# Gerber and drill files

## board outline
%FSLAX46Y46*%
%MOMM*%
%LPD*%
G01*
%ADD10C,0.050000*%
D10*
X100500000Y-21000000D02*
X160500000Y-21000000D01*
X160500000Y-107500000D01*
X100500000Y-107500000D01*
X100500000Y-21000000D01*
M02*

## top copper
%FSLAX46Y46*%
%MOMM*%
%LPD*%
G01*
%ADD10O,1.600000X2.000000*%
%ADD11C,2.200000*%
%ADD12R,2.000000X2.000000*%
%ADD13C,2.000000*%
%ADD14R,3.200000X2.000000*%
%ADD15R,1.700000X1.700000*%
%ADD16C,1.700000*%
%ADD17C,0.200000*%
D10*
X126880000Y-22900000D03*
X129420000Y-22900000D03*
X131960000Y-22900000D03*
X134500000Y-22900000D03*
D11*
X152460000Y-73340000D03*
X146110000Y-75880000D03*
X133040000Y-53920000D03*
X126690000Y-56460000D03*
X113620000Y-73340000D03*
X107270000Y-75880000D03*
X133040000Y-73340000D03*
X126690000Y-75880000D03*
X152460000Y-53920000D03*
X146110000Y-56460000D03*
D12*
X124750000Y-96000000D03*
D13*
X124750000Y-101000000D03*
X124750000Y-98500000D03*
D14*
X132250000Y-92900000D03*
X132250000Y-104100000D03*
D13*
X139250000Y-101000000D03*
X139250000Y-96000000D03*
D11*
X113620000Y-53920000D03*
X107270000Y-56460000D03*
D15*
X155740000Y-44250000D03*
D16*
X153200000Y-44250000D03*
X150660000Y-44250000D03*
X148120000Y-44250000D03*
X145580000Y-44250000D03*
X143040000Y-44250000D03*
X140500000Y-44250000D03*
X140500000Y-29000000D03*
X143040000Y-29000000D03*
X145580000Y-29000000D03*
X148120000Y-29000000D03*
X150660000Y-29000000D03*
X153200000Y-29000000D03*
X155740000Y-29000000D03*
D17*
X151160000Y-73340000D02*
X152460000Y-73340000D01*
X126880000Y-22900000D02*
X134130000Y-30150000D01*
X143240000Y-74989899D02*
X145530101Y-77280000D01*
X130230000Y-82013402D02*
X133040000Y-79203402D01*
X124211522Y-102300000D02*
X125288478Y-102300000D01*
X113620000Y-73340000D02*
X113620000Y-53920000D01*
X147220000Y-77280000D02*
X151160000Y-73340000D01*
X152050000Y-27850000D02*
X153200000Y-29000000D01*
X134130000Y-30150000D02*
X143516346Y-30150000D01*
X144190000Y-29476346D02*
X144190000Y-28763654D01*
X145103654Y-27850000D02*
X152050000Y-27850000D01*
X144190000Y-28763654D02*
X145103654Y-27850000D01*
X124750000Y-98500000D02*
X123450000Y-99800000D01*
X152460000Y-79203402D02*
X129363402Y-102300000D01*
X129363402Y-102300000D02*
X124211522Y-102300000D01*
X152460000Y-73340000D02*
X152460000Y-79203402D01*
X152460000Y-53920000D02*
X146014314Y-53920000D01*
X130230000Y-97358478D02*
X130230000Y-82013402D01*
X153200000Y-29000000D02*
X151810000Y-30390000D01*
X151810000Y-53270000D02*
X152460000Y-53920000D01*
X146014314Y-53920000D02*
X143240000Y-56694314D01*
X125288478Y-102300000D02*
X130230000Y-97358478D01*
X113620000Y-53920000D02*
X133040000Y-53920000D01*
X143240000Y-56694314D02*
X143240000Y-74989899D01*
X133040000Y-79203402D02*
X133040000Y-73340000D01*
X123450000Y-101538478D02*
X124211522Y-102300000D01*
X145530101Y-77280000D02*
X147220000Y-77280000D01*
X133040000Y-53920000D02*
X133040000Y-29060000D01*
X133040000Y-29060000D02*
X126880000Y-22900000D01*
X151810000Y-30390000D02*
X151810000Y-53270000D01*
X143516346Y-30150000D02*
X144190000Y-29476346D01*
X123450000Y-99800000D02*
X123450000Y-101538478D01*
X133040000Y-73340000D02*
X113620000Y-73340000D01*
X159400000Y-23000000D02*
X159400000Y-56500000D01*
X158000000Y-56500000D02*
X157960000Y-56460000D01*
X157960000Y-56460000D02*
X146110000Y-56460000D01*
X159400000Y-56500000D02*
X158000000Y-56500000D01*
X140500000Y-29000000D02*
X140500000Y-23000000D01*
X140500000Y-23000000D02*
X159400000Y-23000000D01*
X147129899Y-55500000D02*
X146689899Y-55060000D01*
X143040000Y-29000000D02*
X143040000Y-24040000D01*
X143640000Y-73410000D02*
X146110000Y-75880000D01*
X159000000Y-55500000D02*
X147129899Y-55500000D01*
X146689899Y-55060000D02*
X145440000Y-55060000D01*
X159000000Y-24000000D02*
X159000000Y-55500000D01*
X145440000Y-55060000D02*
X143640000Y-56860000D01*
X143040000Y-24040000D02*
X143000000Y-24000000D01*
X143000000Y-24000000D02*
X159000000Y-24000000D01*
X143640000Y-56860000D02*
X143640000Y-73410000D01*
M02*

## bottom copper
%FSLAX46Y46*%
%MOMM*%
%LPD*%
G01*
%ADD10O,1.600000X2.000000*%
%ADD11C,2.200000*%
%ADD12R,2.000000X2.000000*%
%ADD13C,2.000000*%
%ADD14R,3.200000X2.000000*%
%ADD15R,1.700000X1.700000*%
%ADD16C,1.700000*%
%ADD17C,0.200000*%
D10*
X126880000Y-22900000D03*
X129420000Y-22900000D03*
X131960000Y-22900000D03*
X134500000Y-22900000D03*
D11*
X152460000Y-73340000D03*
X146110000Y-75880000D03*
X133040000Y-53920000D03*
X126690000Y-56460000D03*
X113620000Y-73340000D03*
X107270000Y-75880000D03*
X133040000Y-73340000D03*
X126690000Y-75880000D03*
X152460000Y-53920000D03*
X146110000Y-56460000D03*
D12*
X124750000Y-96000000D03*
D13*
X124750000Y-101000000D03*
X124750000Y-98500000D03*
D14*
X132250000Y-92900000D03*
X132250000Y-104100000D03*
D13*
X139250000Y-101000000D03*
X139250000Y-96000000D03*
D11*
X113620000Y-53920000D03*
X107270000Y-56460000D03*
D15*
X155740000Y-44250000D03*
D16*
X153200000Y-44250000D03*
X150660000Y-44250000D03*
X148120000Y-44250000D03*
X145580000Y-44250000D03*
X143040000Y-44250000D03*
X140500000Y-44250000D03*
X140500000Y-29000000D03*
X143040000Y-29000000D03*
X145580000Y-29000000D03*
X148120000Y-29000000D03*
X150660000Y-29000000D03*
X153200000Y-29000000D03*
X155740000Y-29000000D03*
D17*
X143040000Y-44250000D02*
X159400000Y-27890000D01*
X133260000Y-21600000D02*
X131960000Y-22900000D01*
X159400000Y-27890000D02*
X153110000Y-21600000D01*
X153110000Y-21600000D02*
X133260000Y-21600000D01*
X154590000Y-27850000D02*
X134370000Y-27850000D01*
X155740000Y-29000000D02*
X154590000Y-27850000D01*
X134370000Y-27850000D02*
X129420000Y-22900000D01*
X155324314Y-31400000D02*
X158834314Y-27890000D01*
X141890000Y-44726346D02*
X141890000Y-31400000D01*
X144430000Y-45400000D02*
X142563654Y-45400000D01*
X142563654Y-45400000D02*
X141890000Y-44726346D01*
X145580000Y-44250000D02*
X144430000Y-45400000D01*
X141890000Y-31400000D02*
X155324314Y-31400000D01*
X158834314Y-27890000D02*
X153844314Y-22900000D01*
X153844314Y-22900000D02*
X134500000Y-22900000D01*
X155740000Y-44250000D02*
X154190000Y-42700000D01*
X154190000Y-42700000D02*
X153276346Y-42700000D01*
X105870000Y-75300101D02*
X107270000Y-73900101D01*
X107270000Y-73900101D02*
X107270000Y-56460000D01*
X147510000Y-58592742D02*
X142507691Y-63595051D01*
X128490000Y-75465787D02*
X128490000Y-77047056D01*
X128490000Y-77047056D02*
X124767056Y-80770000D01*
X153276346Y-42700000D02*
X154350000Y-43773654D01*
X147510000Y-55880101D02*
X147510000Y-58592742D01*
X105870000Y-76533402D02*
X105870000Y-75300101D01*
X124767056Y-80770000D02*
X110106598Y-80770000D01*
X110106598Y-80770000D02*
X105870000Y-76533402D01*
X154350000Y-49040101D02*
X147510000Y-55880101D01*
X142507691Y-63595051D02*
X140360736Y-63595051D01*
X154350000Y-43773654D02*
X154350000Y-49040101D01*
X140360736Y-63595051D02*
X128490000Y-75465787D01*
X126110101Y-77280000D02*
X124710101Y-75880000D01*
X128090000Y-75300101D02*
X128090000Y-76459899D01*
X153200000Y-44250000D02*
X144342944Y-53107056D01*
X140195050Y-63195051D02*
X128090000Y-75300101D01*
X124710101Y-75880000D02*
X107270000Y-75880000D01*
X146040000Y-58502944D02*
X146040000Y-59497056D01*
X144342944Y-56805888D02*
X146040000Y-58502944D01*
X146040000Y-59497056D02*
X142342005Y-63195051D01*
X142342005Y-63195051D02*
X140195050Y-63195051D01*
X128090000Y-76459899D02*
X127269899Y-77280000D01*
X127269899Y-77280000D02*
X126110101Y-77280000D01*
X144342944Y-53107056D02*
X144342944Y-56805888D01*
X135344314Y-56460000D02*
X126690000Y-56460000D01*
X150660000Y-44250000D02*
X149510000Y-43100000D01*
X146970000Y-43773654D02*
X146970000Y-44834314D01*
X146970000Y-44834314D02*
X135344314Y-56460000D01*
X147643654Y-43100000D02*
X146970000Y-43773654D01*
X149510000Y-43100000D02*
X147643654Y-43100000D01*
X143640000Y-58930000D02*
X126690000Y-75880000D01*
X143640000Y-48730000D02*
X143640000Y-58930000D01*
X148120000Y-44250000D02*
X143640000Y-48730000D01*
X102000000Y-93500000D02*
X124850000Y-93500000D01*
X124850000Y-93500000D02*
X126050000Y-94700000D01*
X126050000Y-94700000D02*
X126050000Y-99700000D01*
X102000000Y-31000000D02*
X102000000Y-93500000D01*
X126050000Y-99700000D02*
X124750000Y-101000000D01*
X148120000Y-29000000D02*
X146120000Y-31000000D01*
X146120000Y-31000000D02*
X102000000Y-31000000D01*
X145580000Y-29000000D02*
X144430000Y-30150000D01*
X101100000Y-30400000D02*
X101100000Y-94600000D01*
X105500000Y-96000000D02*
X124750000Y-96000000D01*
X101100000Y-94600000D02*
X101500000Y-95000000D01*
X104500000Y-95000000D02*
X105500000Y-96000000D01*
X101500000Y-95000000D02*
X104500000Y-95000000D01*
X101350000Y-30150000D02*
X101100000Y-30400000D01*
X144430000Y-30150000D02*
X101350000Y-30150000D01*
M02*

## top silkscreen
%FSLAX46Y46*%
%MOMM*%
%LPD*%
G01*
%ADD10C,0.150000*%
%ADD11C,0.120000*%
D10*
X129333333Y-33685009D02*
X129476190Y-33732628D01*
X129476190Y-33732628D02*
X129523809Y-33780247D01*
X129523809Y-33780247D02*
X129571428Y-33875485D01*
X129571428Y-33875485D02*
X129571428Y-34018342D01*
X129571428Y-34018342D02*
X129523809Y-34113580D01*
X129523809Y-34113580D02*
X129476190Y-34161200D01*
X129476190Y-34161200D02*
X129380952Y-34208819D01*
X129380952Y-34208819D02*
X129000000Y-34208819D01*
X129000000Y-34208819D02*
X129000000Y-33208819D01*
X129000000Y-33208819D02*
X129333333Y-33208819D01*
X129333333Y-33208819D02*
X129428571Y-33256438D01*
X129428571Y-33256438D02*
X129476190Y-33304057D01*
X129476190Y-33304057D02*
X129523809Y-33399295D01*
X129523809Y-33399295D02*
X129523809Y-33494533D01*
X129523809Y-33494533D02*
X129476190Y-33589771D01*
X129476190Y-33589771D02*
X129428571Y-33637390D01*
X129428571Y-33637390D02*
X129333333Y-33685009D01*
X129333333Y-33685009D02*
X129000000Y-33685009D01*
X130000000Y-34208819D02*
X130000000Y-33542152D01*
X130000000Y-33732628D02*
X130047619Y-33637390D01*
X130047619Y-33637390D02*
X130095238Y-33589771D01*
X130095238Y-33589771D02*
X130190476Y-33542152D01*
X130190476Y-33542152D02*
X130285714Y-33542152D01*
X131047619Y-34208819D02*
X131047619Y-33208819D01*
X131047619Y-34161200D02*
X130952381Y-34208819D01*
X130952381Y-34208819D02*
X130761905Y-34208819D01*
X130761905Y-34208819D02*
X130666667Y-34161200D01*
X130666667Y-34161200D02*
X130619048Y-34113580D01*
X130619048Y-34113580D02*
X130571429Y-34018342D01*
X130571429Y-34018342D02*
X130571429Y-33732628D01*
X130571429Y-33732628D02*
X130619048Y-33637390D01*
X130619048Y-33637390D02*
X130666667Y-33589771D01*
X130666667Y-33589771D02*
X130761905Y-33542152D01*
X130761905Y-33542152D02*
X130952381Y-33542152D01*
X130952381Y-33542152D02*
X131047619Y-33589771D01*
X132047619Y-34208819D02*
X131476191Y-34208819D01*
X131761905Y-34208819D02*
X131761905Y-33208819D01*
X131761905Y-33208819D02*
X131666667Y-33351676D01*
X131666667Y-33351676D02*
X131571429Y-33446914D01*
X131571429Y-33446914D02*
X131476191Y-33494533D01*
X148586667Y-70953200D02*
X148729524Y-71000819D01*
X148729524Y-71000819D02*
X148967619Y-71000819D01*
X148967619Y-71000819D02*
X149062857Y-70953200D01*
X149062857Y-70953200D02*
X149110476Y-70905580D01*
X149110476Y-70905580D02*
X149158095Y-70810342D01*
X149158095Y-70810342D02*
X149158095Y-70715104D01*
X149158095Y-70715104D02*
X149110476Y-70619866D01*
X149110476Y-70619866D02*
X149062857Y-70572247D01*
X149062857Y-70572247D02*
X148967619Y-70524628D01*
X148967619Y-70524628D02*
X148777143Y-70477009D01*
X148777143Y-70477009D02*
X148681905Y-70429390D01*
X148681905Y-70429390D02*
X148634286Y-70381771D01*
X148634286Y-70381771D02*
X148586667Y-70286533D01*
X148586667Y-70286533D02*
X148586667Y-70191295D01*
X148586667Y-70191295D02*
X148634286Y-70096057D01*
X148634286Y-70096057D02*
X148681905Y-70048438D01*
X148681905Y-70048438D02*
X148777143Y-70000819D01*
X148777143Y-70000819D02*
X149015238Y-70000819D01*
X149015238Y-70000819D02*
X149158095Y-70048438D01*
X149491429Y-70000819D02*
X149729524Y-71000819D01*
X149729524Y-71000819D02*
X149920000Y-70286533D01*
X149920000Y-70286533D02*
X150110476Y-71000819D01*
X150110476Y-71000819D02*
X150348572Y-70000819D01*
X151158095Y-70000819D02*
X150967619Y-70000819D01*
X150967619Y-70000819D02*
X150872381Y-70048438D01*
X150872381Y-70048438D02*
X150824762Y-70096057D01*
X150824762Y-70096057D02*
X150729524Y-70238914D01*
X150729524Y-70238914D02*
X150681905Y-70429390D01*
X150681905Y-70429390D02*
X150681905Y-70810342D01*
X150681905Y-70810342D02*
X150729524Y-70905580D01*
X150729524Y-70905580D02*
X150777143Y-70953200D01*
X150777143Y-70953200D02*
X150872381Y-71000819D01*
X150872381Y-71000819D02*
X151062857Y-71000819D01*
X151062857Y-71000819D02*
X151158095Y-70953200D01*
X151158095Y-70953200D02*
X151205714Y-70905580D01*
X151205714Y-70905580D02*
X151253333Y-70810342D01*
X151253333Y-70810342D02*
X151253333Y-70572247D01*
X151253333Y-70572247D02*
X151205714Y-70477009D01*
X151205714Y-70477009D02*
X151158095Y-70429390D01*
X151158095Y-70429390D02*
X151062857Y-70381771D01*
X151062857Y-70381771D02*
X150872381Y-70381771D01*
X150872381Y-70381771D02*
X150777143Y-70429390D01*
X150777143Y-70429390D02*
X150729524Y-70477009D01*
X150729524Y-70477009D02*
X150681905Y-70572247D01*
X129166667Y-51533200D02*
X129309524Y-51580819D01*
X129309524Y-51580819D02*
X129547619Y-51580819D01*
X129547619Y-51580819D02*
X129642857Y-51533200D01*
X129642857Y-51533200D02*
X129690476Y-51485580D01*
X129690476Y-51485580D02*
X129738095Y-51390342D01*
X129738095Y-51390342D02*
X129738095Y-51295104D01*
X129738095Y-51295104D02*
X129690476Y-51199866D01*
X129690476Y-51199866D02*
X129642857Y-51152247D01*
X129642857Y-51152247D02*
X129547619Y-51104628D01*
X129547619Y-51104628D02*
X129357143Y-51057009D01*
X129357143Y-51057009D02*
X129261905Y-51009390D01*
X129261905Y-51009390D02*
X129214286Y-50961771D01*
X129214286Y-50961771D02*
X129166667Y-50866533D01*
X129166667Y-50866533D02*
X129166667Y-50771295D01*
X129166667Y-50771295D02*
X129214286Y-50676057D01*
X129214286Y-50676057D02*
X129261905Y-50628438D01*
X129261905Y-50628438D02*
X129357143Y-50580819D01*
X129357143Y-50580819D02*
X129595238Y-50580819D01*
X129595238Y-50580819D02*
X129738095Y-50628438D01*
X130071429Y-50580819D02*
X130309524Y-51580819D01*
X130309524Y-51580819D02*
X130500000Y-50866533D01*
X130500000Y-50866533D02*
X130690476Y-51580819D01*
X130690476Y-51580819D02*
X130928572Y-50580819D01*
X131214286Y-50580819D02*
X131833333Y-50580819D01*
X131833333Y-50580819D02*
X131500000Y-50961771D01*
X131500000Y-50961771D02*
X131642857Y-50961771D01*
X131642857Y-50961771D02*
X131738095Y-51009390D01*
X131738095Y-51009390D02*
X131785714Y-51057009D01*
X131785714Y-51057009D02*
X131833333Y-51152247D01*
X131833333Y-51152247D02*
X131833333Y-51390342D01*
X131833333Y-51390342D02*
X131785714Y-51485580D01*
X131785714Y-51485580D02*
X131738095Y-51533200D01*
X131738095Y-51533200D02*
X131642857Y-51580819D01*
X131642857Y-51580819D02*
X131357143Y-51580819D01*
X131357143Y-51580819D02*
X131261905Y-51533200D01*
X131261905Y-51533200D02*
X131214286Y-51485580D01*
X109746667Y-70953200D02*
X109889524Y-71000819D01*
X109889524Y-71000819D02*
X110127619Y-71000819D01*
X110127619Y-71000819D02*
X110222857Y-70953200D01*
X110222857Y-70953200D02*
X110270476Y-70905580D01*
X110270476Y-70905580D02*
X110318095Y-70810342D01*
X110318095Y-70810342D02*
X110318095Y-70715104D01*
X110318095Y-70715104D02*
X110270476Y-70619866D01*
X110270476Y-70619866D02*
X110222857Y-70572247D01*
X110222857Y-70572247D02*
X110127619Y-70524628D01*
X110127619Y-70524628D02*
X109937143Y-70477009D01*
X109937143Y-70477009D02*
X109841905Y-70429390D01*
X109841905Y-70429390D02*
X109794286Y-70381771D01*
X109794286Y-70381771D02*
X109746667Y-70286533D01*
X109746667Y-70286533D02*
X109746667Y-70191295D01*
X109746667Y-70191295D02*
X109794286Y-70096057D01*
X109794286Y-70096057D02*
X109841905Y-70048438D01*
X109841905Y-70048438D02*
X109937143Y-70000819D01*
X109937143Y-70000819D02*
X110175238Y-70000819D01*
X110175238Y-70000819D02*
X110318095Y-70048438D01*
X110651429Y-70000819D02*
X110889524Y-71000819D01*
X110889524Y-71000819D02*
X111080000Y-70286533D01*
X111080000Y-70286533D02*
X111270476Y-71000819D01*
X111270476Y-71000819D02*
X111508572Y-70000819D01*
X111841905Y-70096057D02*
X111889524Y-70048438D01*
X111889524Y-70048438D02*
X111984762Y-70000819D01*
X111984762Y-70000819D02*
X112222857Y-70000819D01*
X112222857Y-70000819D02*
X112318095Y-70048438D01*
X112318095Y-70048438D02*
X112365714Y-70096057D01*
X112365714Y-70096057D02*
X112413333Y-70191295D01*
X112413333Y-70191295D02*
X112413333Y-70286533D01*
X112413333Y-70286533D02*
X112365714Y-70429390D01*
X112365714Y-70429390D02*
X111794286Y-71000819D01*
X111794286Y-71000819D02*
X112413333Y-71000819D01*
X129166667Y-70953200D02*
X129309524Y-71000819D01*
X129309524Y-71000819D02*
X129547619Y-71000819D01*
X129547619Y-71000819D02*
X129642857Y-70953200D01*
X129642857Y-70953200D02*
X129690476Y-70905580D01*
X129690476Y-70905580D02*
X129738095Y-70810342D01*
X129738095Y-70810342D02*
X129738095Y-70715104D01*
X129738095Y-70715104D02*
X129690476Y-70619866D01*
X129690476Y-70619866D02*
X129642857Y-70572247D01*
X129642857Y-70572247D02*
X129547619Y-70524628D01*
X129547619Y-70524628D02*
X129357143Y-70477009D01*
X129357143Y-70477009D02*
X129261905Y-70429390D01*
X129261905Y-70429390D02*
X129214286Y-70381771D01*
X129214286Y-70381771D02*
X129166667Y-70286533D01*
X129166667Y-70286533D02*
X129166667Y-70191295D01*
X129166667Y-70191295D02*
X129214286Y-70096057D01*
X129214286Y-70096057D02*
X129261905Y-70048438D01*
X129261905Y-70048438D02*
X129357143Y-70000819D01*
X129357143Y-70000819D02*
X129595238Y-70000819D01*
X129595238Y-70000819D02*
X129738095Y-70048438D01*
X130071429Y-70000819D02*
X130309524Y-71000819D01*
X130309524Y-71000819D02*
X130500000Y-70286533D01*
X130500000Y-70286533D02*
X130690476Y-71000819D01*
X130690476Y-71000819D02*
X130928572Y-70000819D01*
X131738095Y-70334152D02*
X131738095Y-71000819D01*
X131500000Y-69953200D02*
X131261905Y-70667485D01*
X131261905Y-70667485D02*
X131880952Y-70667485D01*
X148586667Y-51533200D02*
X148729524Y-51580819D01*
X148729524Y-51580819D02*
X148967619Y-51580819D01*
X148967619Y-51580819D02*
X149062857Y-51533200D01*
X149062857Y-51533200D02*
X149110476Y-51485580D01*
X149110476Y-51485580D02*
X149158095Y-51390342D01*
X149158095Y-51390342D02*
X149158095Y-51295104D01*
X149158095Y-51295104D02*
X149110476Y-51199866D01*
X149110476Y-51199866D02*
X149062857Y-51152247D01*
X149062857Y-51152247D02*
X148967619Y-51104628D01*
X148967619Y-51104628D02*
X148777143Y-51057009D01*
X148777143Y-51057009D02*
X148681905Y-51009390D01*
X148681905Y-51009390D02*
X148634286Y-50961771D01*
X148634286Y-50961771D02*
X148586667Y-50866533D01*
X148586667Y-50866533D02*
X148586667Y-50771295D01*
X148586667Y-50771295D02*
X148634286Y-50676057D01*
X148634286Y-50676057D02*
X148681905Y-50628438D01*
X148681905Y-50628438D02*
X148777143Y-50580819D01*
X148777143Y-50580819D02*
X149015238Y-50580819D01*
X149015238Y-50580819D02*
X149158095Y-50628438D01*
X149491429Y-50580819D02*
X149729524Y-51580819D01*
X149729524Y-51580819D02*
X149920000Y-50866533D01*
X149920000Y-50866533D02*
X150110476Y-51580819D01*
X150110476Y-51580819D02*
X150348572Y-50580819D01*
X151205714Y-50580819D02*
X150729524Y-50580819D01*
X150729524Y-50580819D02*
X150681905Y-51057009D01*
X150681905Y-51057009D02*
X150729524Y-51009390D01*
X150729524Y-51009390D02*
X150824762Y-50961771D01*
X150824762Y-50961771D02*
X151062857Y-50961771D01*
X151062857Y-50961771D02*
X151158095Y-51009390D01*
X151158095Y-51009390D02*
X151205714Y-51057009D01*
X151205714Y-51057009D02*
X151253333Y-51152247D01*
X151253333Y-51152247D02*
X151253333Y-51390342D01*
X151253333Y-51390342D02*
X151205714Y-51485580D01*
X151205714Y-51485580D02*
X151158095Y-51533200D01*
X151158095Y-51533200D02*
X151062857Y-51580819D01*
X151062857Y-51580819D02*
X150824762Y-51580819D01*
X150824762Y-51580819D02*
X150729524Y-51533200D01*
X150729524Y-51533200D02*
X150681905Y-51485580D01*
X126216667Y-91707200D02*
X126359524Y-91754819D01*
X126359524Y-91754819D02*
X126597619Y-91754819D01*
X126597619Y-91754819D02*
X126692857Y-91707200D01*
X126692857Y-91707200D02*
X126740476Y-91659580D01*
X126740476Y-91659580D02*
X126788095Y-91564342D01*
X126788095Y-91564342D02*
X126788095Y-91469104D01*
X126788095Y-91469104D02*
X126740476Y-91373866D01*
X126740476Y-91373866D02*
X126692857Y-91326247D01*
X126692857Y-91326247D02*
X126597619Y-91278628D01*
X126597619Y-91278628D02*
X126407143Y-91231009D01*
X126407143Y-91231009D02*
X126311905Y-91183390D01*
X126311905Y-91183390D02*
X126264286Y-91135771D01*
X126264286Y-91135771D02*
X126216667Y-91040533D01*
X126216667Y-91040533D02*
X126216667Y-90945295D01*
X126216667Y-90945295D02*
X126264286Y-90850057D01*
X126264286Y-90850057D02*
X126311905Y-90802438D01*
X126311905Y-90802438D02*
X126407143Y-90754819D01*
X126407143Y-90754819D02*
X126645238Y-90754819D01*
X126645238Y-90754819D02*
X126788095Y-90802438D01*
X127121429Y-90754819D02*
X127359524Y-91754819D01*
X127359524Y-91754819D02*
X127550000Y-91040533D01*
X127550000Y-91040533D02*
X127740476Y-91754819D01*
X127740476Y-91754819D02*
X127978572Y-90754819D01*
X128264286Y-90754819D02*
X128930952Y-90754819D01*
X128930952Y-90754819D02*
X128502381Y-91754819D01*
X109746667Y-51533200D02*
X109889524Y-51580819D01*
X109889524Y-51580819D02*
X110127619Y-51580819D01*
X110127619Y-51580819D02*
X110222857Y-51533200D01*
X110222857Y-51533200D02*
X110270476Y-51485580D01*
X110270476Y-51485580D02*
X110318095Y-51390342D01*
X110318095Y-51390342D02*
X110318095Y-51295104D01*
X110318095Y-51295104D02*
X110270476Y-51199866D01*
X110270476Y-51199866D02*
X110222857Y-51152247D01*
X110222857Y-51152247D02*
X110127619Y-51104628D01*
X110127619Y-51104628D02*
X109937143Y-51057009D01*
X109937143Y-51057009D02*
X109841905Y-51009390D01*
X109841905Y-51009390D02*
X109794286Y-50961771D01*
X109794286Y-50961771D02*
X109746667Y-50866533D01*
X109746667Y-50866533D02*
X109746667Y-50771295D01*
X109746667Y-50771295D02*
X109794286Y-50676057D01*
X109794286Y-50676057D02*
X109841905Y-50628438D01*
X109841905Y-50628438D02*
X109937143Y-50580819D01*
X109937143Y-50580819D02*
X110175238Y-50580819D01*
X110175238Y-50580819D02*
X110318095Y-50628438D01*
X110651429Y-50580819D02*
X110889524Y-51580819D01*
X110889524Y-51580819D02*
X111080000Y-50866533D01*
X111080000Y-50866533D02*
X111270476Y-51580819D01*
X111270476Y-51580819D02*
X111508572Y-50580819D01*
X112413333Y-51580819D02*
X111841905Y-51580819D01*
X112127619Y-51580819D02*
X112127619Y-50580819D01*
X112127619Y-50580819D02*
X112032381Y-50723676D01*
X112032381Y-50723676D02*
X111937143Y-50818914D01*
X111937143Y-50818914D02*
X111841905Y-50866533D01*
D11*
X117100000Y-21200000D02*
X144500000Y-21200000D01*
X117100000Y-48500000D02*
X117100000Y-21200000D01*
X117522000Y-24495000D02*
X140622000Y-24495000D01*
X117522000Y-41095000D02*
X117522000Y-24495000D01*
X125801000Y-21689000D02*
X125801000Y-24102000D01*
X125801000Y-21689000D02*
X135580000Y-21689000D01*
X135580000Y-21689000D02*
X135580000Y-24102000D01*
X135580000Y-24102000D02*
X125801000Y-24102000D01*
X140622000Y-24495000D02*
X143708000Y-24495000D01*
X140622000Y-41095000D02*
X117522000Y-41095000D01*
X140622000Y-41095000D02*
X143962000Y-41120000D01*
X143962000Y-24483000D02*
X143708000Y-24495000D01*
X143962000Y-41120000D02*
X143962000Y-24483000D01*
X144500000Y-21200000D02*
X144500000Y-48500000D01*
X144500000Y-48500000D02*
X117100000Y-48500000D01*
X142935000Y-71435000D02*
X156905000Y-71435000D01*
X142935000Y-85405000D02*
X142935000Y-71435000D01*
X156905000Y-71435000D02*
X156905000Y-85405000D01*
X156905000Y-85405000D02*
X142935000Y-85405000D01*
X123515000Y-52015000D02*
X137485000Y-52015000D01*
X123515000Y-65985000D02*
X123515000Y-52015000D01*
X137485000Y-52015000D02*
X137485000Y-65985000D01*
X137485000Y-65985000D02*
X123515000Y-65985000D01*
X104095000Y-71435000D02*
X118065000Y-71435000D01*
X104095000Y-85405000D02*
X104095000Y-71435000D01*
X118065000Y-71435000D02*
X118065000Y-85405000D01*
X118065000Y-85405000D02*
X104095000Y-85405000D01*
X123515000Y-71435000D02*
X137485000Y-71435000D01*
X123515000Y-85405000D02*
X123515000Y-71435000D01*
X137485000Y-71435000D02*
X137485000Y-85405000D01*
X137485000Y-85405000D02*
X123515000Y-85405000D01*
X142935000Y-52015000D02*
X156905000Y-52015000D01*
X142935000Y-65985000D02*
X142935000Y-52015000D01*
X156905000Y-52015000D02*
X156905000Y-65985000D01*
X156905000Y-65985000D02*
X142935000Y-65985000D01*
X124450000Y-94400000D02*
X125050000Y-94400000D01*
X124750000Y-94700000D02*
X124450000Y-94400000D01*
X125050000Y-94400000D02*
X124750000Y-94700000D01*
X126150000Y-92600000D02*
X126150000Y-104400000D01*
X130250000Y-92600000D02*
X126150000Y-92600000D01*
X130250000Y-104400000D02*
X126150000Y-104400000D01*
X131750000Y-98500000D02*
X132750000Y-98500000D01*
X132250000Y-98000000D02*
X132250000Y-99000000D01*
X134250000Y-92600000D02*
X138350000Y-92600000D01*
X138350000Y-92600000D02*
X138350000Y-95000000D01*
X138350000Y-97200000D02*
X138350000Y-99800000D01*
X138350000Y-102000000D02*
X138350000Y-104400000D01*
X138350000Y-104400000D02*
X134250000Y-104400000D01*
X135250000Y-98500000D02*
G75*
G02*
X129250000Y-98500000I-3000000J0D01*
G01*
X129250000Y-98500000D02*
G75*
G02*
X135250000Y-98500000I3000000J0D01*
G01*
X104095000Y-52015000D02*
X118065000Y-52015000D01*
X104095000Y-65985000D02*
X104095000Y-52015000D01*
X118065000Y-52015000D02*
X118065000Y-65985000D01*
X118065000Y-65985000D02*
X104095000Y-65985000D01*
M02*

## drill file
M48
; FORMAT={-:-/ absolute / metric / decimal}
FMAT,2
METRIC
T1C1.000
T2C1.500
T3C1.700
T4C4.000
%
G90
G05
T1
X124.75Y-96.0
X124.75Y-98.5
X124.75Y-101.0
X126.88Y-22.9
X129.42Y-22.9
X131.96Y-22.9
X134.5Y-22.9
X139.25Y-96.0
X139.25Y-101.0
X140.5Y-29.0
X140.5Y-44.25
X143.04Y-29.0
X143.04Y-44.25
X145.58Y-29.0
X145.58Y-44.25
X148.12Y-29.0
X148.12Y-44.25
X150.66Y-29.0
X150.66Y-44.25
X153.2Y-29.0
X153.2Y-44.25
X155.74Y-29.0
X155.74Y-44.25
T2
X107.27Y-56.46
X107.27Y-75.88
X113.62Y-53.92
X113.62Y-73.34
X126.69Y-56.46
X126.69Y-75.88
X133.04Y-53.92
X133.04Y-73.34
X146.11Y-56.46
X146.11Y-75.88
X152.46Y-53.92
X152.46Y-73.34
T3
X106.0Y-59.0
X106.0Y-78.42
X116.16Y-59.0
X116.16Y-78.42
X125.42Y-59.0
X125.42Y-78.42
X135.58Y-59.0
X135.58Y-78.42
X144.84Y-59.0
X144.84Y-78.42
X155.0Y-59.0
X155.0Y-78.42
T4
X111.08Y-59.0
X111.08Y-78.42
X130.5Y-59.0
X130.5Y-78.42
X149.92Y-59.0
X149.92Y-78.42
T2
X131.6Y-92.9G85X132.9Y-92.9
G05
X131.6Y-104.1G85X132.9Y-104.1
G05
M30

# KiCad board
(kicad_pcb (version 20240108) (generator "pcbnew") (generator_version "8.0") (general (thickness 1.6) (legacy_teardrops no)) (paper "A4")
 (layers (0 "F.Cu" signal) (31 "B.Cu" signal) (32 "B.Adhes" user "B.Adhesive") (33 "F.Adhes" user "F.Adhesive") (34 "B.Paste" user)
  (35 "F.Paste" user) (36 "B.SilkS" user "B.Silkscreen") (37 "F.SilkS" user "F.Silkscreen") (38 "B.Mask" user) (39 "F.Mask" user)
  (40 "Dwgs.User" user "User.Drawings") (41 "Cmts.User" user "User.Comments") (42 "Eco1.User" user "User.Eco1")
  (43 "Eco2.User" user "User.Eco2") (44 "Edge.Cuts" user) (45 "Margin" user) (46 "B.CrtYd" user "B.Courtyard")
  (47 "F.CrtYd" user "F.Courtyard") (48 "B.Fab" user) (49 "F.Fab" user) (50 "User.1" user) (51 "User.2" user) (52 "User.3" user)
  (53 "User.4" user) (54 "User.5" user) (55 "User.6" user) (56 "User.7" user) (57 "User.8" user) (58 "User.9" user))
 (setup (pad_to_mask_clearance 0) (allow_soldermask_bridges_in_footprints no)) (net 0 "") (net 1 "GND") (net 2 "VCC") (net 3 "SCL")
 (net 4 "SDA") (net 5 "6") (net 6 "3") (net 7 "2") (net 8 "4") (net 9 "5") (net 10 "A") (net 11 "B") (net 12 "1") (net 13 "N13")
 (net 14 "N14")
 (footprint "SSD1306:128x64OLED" (layer "F.Cu") (at 130.5 33.5)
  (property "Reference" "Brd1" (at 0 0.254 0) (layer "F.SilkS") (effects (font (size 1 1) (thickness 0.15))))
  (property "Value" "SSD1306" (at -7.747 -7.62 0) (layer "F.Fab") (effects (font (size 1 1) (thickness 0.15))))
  (fp_line (start -13.4 -12.3) (end 14 -12.3) (stroke (width 0.12) (type solid)) (layer "F.SilkS"))
  (fp_line (start -13.4 15) (end -13.4 -12.3) (stroke (width 0.12) (type solid)) (layer "F.SilkS"))
  (fp_line (start -12.978 -9.005) (end 10.122 -9.005) (stroke (width 0.12) (type solid)) (layer "F.SilkS"))
  (fp_line (start -12.978 7.595) (end -12.978 -9.005) (stroke (width 0.12) (type solid)) (layer "F.SilkS"))
  (fp_line (start -4.699 -11.811) (end -4.699 -9.398) (stroke (width 0.12) (type solid)) (layer "F.SilkS"))
  (fp_line (start -4.699 -11.811) (end 5.08 -11.811) (stroke (width 0.12) (type solid)) (layer "F.SilkS"))
  (fp_line (start 5.08 -11.811) (end 5.08 -9.398) (stroke (width 0.12) (type solid)) (layer "F.SilkS"))
  (fp_line (start 5.08 -9.398) (end -4.699 -9.398) (stroke (width 0.12) (type solid)) (layer "F.SilkS"))
  (fp_line (start 10.122 -9.005) (end 13.208 -9.005) (stroke (width 0.12) (type solid)) (layer "F.SilkS"))
  (fp_line (start 10.122 7.595) (end -12.978 7.595) (stroke (width 0.12) (type solid)) (layer "F.SilkS"))
  (fp_line (start 10.122 7.595) (end 13.462 7.62) (stroke (width 0.12) (type solid)) (layer "F.SilkS"))
  (fp_line (start 13.462 -9.017) (end 13.208 -9.005) (stroke (width 0.12) (type solid)) (layer "F.SilkS"))
  (fp_line (start 13.462 7.62) (end 13.462 -9.017) (stroke (width 0.12) (type solid)) (layer "F.SilkS"))
  (fp_line (start 14 -12.3) (end 14 15) (stroke (width 0.12) (type solid)) (layer "F.SilkS"))
  (fp_line (start 14 15) (end -13.4 15) (stroke (width 0.12) (type solid)) (layer "F.SilkS"))
  (pad "1" thru_hole oval (at -3.62 -10.6 90) (size 2 1.6) (drill 1) (layers "*.Cu" "*.Mask") (remove_unused_layers no) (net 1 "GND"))
  (pad "2" thru_hole oval (at -1.08 -10.6 90) (size 2 1.6) (drill 1) (layers "*.Cu" "*.Mask") (remove_unused_layers no) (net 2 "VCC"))
  (pad "3" thru_hole oval (at 1.46 -10.6 90) (size 2 1.6) (drill 1) (layers "*.Cu" "*.Mask") (remove_unused_layers no) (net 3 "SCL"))
  (pad "4" thru_hole oval (at 4 -10.6 90) (size 2 1.6) (drill 1) (layers "*.Cu" "*.Mask") (remove_unused_layers no) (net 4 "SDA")))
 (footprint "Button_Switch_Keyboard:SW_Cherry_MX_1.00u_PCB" (layer "F.Cu") (at 152.46 73.34)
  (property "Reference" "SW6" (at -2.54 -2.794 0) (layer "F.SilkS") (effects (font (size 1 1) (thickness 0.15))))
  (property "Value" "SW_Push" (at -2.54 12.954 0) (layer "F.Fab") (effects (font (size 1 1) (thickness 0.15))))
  (fp_line (start -9.525 -1.905) (end 4.445 -1.905) (stroke (width 0.12) (type solid)) (layer "F.SilkS"))
  (fp_line (start -9.525 12.065) (end -9.525 -1.905) (stroke (width 0.12) (type solid)) (layer "F.SilkS"))
  (fp_line (start 4.445 -1.905) (end 4.445 12.065) (stroke (width 0.12) (type solid)) (layer "F.SilkS"))
  (fp_line (start 4.445 12.065) (end -9.525 12.065) (stroke (width 0.12) (type solid)) (layer "F.SilkS"))
  (pad "" np_thru_hole circle (at -7.62 5.08) (size 1.7 1.7) (drill 1.7) (layers "*.Cu" "*.Mask"))
  (pad "" np_thru_hole circle (at -2.54 5.08) (size 4 4) (drill 4) (layers "*.Cu" "*.Mask"))
  (pad "" np_thru_hole circle (at 2.54 5.08) (size 1.7 1.7) (drill 1.7) (layers "*.Cu" "*.Mask"))
  (pad "1" thru_hole circle (at 0 0) (size 2.2 2.2) (drill 1.5) (layers "*.Cu" "*.Mask") (remove_unused_layers no) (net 1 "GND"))
  (pad "2" thru_hole circle (at -6.35 2.54) (size 2.2 2.2) (drill 1.5) (layers "*.Cu" "*.Mask") (remove_unused_layers no) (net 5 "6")))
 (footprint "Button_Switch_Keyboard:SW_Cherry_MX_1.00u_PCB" (layer "F.Cu") (at 133.04 53.92)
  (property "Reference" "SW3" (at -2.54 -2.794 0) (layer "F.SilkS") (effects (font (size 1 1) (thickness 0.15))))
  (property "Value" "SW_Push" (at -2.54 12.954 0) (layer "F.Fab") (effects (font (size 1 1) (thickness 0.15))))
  (fp_line (start -9.525 -1.905) (end 4.445 -1.905) (stroke (width 0.12) (type solid)) (layer "F.SilkS"))
  (fp_line (start -9.525 12.065) (end -9.525 -1.905) (stroke (width 0.12) (type solid)) (layer "F.SilkS"))
  (fp_line (start 4.445 -1.905) (end 4.445 12.065) (stroke (width 0.12) (type solid)) (layer "F.SilkS"))
  (fp_line (start 4.445 12.065) (end -9.525 12.065) (stroke (width 0.12) (type solid)) (layer "F.SilkS"))
  (pad "" np_thru_hole circle (at -7.62 5.08) (size 1.7 1.7) (drill 1.7) (layers "*.Cu" "*.Mask"))
  (pad "" np_thru_hole circle (at -2.54 5.08) (size 4 4) (drill 4) (layers "*.Cu" "*.Mask"))
  (pad "" np_thru_hole circle (at 2.54 5.08) (size 1.7 1.7) (drill 1.7) (layers "*.Cu" "*.Mask"))
  (pad "1" thru_hole circle (at 0 0) (size 2.2 2.2) (drill 1.5) (layers "*.Cu" "*.Mask") (remove_unused_layers no) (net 1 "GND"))
  (pad "2" thru_hole circle (at -6.35 2.54) (size 2.2 2.2) (drill 1.5) (layers "*.Cu" "*.Mask") (remove_unused_layers no) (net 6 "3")))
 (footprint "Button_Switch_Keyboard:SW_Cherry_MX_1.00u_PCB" (layer "F.Cu") (at 113.62 73.34)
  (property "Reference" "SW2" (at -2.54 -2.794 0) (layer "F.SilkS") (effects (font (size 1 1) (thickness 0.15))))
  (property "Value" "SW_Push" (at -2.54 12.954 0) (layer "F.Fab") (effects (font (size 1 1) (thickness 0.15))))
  (fp_line (start -9.525 -1.905) (end 4.445 -1.905) (stroke (width 0.12) (type solid)) (layer "F.SilkS"))
  (fp_line (start -9.525 12.065) (end -9.525 -1.905) (stroke (width 0.12) (type solid)) (layer "F.SilkS"))
  (fp_line (start 4.445 -1.905) (end 4.445 12.065) (stroke (width 0.12) (type solid)) (layer "F.SilkS"))
  (fp_line (start 4.445 12.065) (end -9.525 12.065) (stroke (width 0.12) (type solid)) (layer "F.SilkS"))
  (pad "" np_thru_hole circle (at -7.62 5.08) (size 1.7 1.7) (drill 1.7) (layers "*.Cu" "*.Mask"))
  (pad "" np_thru_hole circle (at -2.54 5.08) (size 4 4) (drill 4) (layers "*.Cu" "*.Mask"))
  (pad "" np_thru_hole circle (at 2.54 5.08) (size 1.7 1.7) (drill 1.7) (layers "*.Cu" "*.Mask"))
  (pad "1" thru_hole circle (at 0 0) (size 2.2 2.2) (drill 1.5) (layers "*.Cu" "*.Mask") (remove_unused_layers no) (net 1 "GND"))
  (pad "2" thru_hole circle (at -6.35 2.54) (size 2.2 2.2) (drill 1.5) (layers "*.Cu" "*.Mask") (remove_unused_layers no) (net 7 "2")))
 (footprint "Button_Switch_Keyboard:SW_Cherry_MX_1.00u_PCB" (layer "F.Cu") (at 133.04 73.34)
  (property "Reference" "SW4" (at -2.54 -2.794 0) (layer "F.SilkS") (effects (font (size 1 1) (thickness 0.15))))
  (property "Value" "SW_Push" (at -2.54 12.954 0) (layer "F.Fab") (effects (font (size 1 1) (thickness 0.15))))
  (fp_line (start -9.525 -1.905) (end 4.445 -1.905) (stroke (width 0.12) (type solid)) (layer "F.SilkS"))
  (fp_line (start -9.525 12.065) (end -9.525 -1.905) (stroke (width 0.12) (type solid)) (layer "F.SilkS"))
  (fp_line (start 4.445 -1.905) (end 4.445 12.065) (stroke (width 0.12) (type solid)) (layer "F.SilkS"))
  (fp_line (start 4.445 12.065) (end -9.525 12.065) (stroke (width 0.12) (type solid)) (layer "F.SilkS"))
  (pad "" np_thru_hole circle (at -7.62 5.08) (size 1.7 1.7) (drill 1.7) (layers "*.Cu" "*.Mask"))
  (pad "" np_thru_hole circle (at -2.54 5.08) (size 4 4) (drill 4) (layers "*.Cu" "*.Mask"))
  (pad "" np_thru_hole circle (at 2.54 5.08) (size 1.7 1.7) (drill 1.7) (layers "*.Cu" "*.Mask"))
  (pad "1" thru_hole circle (at 0 0) (size 2.2 2.2) (drill 1.5) (layers "*.Cu" "*.Mask") (remove_unused_layers no) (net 1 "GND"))
  (pad "2" thru_hole circle (at -6.35 2.54) (size 2.2 2.2) (drill 1.5) (layers "*.Cu" "*.Mask") (remove_unused_layers no) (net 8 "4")))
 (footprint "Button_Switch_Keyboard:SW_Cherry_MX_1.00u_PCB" (layer "F.Cu") (at 152.46 53.92)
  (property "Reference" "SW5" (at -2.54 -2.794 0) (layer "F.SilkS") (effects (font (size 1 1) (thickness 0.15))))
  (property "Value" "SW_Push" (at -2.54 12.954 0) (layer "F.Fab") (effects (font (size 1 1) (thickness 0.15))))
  (fp_line (start -9.525 -1.905) (end 4.445 -1.905) (stroke (width 0.12) (type solid)) (layer "F.SilkS"))
  (fp_line (start -9.525 12.065) (end -9.525 -1.905) (stroke (width 0.12) (type solid)) (layer "F.SilkS"))
  (fp_line (start 4.445 -1.905) (end 4.445 12.065) (stroke (width 0.12) (type solid)) (layer "F.SilkS"))
  (fp_line (start 4.445 12.065) (end -9.525 12.065) (stroke (width 0.12) (type solid)) (layer "F.SilkS"))
  (pad "" np_thru_hole circle (at -7.62 5.08) (size 1.7 1.7) (drill 1.7) (layers "*.Cu" "*.Mask"))
  (pad "" np_thru_hole circle (at -2.54 5.08) (size 4 4) (drill 4) (layers "*.Cu" "*.Mask"))
  (pad "" np_thru_hole circle (at 2.54 5.08) (size 1.7 1.7) (drill 1.7) (layers "*.Cu" "*.Mask"))
  (pad "1" thru_hole circle (at 0 0) (size 2.2 2.2) (drill 1.5) (layers "*.Cu" "*.Mask") (remove_unused_layers no) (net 1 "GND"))
  (pad "2" thru_hole circle (at -6.35 2.54) (size 2.2 2.2) (drill 1.5) (layers "*.Cu" "*.Mask") (remove_unused_layers no) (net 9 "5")))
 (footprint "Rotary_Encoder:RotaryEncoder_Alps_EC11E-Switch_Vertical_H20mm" (layer "F.Cu") (at 124.75 96)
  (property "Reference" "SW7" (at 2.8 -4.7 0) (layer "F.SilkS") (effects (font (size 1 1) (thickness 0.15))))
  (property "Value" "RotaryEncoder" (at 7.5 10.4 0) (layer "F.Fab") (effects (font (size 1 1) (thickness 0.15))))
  (fp_line (start -0.3 -1.6) (end 0.3 -1.6) (stroke (width 0.12) (type solid)) (layer "F.SilkS"))
  (fp_line (start 0 -1.3) (end -0.3 -1.6) (stroke (width 0.12) (type solid)) (layer "F.SilkS"))
  (fp_line (start 0.3 -1.6) (end 0 -1.3) (stroke (width 0.12) (type solid)) (layer "F.SilkS"))
  (fp_line (start 1.4 -3.4) (end 1.4 8.4) (stroke (width 0.12) (type solid)) (layer "F.SilkS"))
  (fp_line (start 5.5 -3.4) (end 1.4 -3.4) (stroke (width 0.12) (type solid)) (layer "F.SilkS"))
  (fp_line (start 5.5 8.4) (end 1.4 8.4) (stroke (width 0.12) (type solid)) (layer "F.SilkS"))
  (fp_line (start 7 2.5) (end 8 2.5) (stroke (width 0.12) (type solid)) (layer "F.SilkS"))
  (fp_line (start 7.5 2) (end 7.5 3) (stroke (width 0.12) (type solid)) (layer "F.SilkS"))
  (fp_line (start 9.5 -3.4) (end 13.6 -3.4) (stroke (width 0.12) (type solid)) (layer "F.SilkS"))
  (fp_line (start 13.6 -3.4) (end 13.6 -1) (stroke (width 0.12) (type solid)) (layer "F.SilkS"))
  (fp_line (start 13.6 1.2) (end 13.6 3.8) (stroke (width 0.12) (type solid)) (layer "F.SilkS"))
  (fp_line (start 13.6 6) (end 13.6 8.4) (stroke (width 0.12) (type solid)) (layer "F.SilkS"))
  (fp_line (start 13.6 8.4) (end 9.5 8.4) (stroke (width 0.12) (type solid)) (layer "F.SilkS"))
  (fp_circle (center 7.5 2.5) (end 10.5 2.5) (stroke (width 0.12) (type solid)) (fill none) (layer "F.SilkS"))
  (pad "A" thru_hole rect (at 0 0) (size 2 2) (drill 1) (layers "*.Cu" "*.Mask") (remove_unused_layers no) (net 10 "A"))
  (pad "B" thru_hole circle (at 0 5) (size 2 2) (drill 1) (layers "*.Cu" "*.Mask") (remove_unused_layers no) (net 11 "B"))
  (pad "C" thru_hole circle (at 0 2.5) (size 2 2) (drill 1) (layers "*.Cu" "*.Mask") (remove_unused_layers no) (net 1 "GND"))
  (pad "MP" thru_hole rect (at 7.5 -3.1) (size 3.2 2) (drill oval 2.8 1.5) (layers "*.Cu" "*.Mask") (remove_unused_layers no))
  (pad "MP" thru_hole rect (at 7.5 8.1) (size 3.2 2) (drill oval 2.8 1.5) (layers "*.Cu" "*.Mask") (remove_unused_layers no))
  (pad "S1" thru_hole circle (at 14.5 5) (size 2 2) (drill 1) (layers "*.Cu" "*.Mask") (remove_unused_layers no))
  (pad "S2" thru_hole circle (at 14.5 0) (size 2 2) (drill 1) (layers "*.Cu" "*.Mask") (remove_unused_layers no)))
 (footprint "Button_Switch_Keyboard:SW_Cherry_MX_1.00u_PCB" (layer "F.Cu") (at 113.62 53.92)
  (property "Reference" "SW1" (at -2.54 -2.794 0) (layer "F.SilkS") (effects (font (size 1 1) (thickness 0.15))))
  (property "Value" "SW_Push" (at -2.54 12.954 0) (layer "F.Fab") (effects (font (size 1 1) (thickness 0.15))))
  (fp_line (start -9.525 -1.905) (end 4.445 -1.905) (stroke (width 0.12) (type solid)) (layer "F.SilkS"))
  (fp_line (start -9.525 12.065) (end -9.525 -1.905) (stroke (width 0.12) (type solid)) (layer "F.SilkS"))
  (fp_line (start 4.445 -1.905) (end 4.445 12.065) (stroke (width 0.12) (type solid)) (layer "F.SilkS"))
  (fp_line (start 4.445 12.065) (end -9.525 12.065) (stroke (width 0.12) (type solid)) (layer "F.SilkS"))
  (pad "" np_thru_hole circle (at -7.62 5.08) (size 1.7 1.7) (drill 1.7) (layers "*.Cu" "*.Mask"))
  (pad "" np_thru_hole circle (at -2.54 5.08) (size 4 4) (drill 4) (layers "*.Cu" "*.Mask"))
  (pad "" np_thru_hole circle (at 2.54 5.08) (size 1.7 1.7) (drill 1.7) (layers "*.Cu" "*.Mask"))
  (pad "1" thru_hole circle (at 0 0) (size 2.2 2.2) (drill 1.5) (layers "*.Cu" "*.Mask") (remove_unused_layers no) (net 1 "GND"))
  (pad "2" thru_hole circle (at -6.35 2.54) (size 2.2 2.2) (drill 1.5) (layers "*.Cu" "*.Mask") (remove_unused_layers no) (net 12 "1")))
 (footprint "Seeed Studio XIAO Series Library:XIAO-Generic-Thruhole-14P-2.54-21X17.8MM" (layer "B.Cu") (at 148.12 36.625 90)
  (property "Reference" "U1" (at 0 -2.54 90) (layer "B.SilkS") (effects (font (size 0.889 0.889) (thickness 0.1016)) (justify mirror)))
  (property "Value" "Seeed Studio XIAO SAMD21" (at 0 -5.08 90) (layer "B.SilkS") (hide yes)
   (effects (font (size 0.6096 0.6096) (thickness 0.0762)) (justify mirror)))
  (pad "1" thru_hole rect (at -7.625 7.62 90) (size 1.7 1.7) (drill 1) (layers "*.Cu" "*.Mask") (remove_unused_layers no) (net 12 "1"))
  (pad "2" thru_hole circle (at -7.625 5.08 90) (size 1.7 1.7) (drill 1) (layers "*.Cu" "*.Mask") (remove_unused_layers no) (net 7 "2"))
  (pad "3" thru_hole circle (at -7.625 2.54 90) (size 1.7 1.7) (drill 1) (layers "*.Cu" "*.Mask") (remove_unused_layers no) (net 6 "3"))
  (pad "4" thru_hole circle (at -7.625 0 90) (size 1.7 1.7) (drill 1) (layers "*.Cu" "*.Mask") (remove_unused_layers no) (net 8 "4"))
  (pad "5" thru_hole circle (at -7.625 -2.54 90) (size 1.7 1.7) (drill 1) (layers "*.Cu" "*.Mask") (remove_unused_layers no) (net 4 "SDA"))
  (pad "6" thru_hole circle (at -7.625 -5.08 270) (size 1.7 1.7) (drill 1) (layers "*.Cu" "*.Mask") (remove_unused_layers no) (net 3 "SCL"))
  (pad "7" thru_hole circle (at -7.625 -7.62 90) (size 1.7 1.7) (drill 1) (layers "*.Cu" "*.Mask") (remove_unused_layers no) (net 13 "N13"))
  (pad "8" thru_hole circle (at 7.625 -7.62 90) (size 1.7 1.7) (drill 1) (layers "*.Cu" "*.Mask") (remove_unused_layers no) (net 9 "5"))
  (pad "9" thru_hole circle (at 7.625 -5.08 90) (size 1.7 1.7) (drill 1) (layers "*.Cu" "*.Mask") (remove_unused_layers no) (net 5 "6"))
  (pad "10" thru_hole circle (at 7.625 -2.54 90) (size 1.7 1.7) (drill 1) (layers "*.Cu" "*.Mask") (remove_unused_layers no) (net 10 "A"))
  (pad "11" thru_hole circle (at 7.625 0 90) (size 1.7 1.7) (drill 1) (layers "*.Cu" "*.Mask") (remove_unused_layers no) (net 11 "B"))
  (pad "12" thru_hole circle (at 7.625 2.54 90) (size 1.7 1.7) (drill 1) (layers "*.Cu" "*.Mask") (remove_unused_layers no) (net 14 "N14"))
  (pad "13" thru_hole circle (at 7.625 5.08 90) (size 1.7 1.7) (drill 1) (layers "*.Cu" "*.Mask") (remove_unused_layers no) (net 1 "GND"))
  (pad "14" thru_hole circle (at 7.625 7.62 90) (size 1.7 1.7) (drill 1) (layers "*.Cu" "*.Mask") (remove_unused_layers no) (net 2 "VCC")))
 (gr_rect (start 100.5 21) (end 160.5 107.5) (stroke (width 0.05) (type default)) (fill none) (layer "Edge.Cuts"))
 (segment (start 151.16 73.34) (end 152.46 73.34) (width 0.2) (layer "F.Cu") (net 1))
 (segment (start 126.88 22.9) (end 134.13 30.15) (width 0.2) (layer "F.Cu") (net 1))
 (segment (start 143.24 74.989899) (end 145.530101 77.28) (width 0.2) (layer "F.Cu") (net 1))
 (segment (start 130.23 82.013402) (end 133.04 79.203402) (width 0.2) (layer "F.Cu") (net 1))
 (segment (start 124.211522 102.3) (end 125.288478 102.3) (width 0.2) (layer "F.Cu") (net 1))
 (segment (start 113.62 73.34) (end 113.62 53.92) (width 0.2) (layer "F.Cu") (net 1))
 (segment (start 147.22 77.28) (end 151.16 73.34) (width 0.2) (layer "F.Cu") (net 1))
 (segment (start 152.05 27.85) (end 153.2 29) (width 0.2) (layer "F.Cu") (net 1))
 (segment (start 134.13 30.15) (end 143.516346 30.15) (width 0.2) (layer "F.Cu") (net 1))
 (segment (start 144.19 29.476346) (end 144.19 28.763654) (width 0.2) (layer "F.Cu") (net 1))
 (segment (start 145.103654 27.85) (end 152.05 27.85) (width 0.2) (layer "F.Cu") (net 1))
 (segment (start 144.19 28.763654) (end 145.103654 27.85) (width 0.2) (layer "F.Cu") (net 1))
 (segment (start 124.75 98.5) (end 123.45 99.8) (width 0.2) (layer "F.Cu") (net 1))
 (segment (start 152.46 79.203402) (end 129.363402 102.3) (width 0.2) (layer "F.Cu") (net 1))
 (segment (start 129.363402 102.3) (end 124.211522 102.3) (width 0.2) (layer "F.Cu") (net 1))
 (segment (start 152.46 73.34) (end 152.46 79.203402) (width 0.2) (layer "F.Cu") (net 1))
 (segment (start 152.46 53.92) (end 146.014314 53.92) (width 0.2) (layer "F.Cu") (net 1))
 (segment (start 130.23 97.358478) (end 130.23 82.013402) (width 0.2) (layer "F.Cu") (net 1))
 (segment (start 153.2 29) (end 151.81 30.39) (width 0.2) (layer "F.Cu") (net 1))
 (segment (start 151.81 53.27) (end 152.46 53.92) (width 0.2) (layer "F.Cu") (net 1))
 (segment (start 146.014314 53.92) (end 143.24 56.694314) (width 0.2) (layer "F.Cu") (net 1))
 (segment (start 125.288478 102.3) (end 130.23 97.358478) (width 0.2) (layer "F.Cu") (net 1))
 (segment (start 113.62 53.92) (end 133.04 53.92) (width 0.2) (layer "F.Cu") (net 1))
 (segment (start 143.24 56.694314) (end 143.24 74.989899) (width 0.2) (layer "F.Cu") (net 1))
 (segment (start 133.04 79.203402) (end 133.04 73.34) (width 0.2) (layer "F.Cu") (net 1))
 (segment (start 123.45 101.538478) (end 124.211522 102.3) (width 0.2) (layer "F.Cu") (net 1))
 (segment (start 145.530101 77.28) (end 147.22 77.28) (width 0.2) (layer "F.Cu") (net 1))
 (segment (start 133.04 53.92) (end 133.04 29.06) (width 0.2) (layer "F.Cu") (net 1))
 (segment (start 133.04 29.06) (end 126.88 22.9) (width 0.2) (layer "F.Cu") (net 1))
 (segment (start 151.81 30.39) (end 151.81 53.27) (width 0.2) (layer "F.Cu") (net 1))
 (segment (start 143.516346 30.15) (end 144.19 29.476346) (width 0.2) (layer "F.Cu") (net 1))
 (segment (start 123.45 99.8) (end 123.45 101.538478) (width 0.2) (layer "F.Cu") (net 1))
 (segment (start 133.04 73.34) (end 113.62 73.34) (width 0.2) (layer "F.Cu") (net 1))
 (segment (start 143.04 44.25) (end 159.4 27.89) (width 0.2) (layer "B.Cu") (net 3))
 (segment (start 133.26 21.6) (end 131.96 22.9) (width 0.2) (layer "B.Cu") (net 3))
 (segment (start 159.4 27.89) (end 153.11 21.6) (width 0.2) (layer "B.Cu") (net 3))
 (segment (start 153.11 21.6) (end 133.26 21.6) (width 0.2) (layer "B.Cu") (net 3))
 (segment (start 154.59 27.85) (end 134.37 27.85) (width 0.2) (layer "B.Cu") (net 2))
 (segment (start 155.74 29) (end 154.59 27.85) (width 0.2) (layer "B.Cu") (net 2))
 (segment (start 134.37 27.85) (end 129.42 22.9) (width 0.2) (layer "B.Cu") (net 2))
 (segment (start 155.324314 31.4) (end 158.834314 27.89) (width 0.2) (layer "B.Cu") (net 4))
 (segment (start 141.89 44.726346) (end 141.89 31.4) (width 0.2) (layer "B.Cu") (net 4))
 (segment (start 144.43 45.4) (end 142.563654 45.4) (width 0.2) (layer "B.Cu") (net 4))
 (segment (start 142.563654 45.4) (end 141.89 44.726346) (width 0.2) (layer "B.Cu") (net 4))
 (segment (start 145.58 44.25) (end 144.43 45.4) (width 0.2) (layer "B.Cu") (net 4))
 (segment (start 141.89 31.4) (end 155.324314 31.4) (width 0.2) (layer "B.Cu") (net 4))
 (segment (start 158.834314 27.89) (end 153.844314 22.9) (width 0.2) (layer "B.Cu") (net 4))
 (segment (start 153.844314 22.9) (end 134.5 22.9) (width 0.2) (layer "B.Cu") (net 4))
 (segment (start 155.74 44.25) (end 154.19 42.7) (width 0.2) (layer "B.Cu") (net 12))
 (segment (start 154.19 42.7) (end 153.276346 42.7) (width 0.2) (layer "B.Cu") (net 12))
 (segment (start 105.87 75.300101) (end 107.27 73.900101) (width 0.2) (layer "B.Cu") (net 12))
 (segment (start 107.27 73.900101) (end 107.27 56.46) (width 0.2) (layer "B.Cu") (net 12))
 (segment (start 147.51 58.592742) (end 142.507691 63.595051) (width 0.2) (layer "B.Cu") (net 12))
 (segment (start 128.49 75.465787) (end 128.49 77.047056) (width 0.2) (layer "B.Cu") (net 12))
 (segment (start 128.49 77.047056) (end 124.767056 80.77) (width 0.2) (layer "B.Cu") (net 12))
 (segment (start 153.276346 42.7) (end 154.35 43.773654) (width 0.2) (layer "B.Cu") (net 12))
 (segment (start 147.51 55.880101) (end 147.51 58.592742) (width 0.2) (layer "B.Cu") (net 12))
 (segment (start 105.87 76.533402) (end 105.87 75.300101) (width 0.2) (layer "B.Cu") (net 12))
 (segment (start 124.767056 80.77) (end 110.106598 80.77) (width 0.2) (layer "B.Cu") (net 12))
 (segment (start 110.106598 80.77) (end 105.87 76.533402) (width 0.2) (layer "B.Cu") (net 12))
 (segment (start 154.35 49.040101) (end 147.51 55.880101) (width 0.2) (layer "B.Cu") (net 12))
 (segment (start 142.507691 63.595051) (end 140.360736 63.595051) (width 0.2) (layer "B.Cu") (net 12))
 (segment (start 154.35 43.773654) (end 154.35 49.040101) (width 0.2) (layer "B.Cu") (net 12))
 (segment (start 140.360736 63.595051) (end 128.49 75.465787) (width 0.2) (layer "B.Cu") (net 12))
 (segment (start 126.110101 77.28) (end 124.710101 75.88) (width 0.2) (layer "B.Cu") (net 7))
 (segment (start 128.09 75.300101) (end 128.09 76.459899) (width 0.2) (layer "B.Cu") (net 7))
 (segment (start 153.2 44.25) (end 144.342944 53.107056) (width 0.2) (layer "B.Cu") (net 7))
 (segment (start 140.19505 63.195051) (end 128.09 75.300101) (width 0.2) (layer "B.Cu") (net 7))
 (segment (start 124.710101 75.88) (end 107.27 75.88) (width 0.2) (layer "B.Cu") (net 7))
 (segment (start 146.04 58.502944) (end 146.04 59.497056) (width 0.2) (layer "B.Cu") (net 7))
 (segment (start 144.342944 56.805888) (end 146.04 58.502944) (width 0.2) (layer "B.Cu") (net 7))
 (segment (start 146.04 59.497056) (end 142.342005 63.195051) (width 0.2) (layer "B.Cu") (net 7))
 (segment (start 142.342005 63.195051) (end 140.19505 63.195051) (width 0.2) (layer "B.Cu") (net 7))
 (segment (start 128.09 76.459899) (end 127.269899 77.28) (width 0.2) (layer "B.Cu") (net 7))
 (segment (start 127.269899 77.28) (end 126.110101 77.28) (width 0.2) (layer "B.Cu") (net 7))
 (segment (start 144.342944 53.107056) (end 144.342944 56.805888) (width 0.2) (layer "B.Cu") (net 7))
 (segment (start 135.344314 56.46) (end 126.69 56.46) (width 0.2) (layer "B.Cu") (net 6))
 (segment (start 150.66 44.25) (end 149.51 43.1) (width 0.2) (layer "B.Cu") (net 6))
 (segment (start 146.97 43.773654) (end 146.97 44.834314) (width 0.2) (layer "B.Cu") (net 6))
 (segment (start 146.97 44.834314) (end 135.344314 56.46) (width 0.2) (layer "B.Cu") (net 6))
 (segment (start 147.643654 43.1) (end 146.97 43.773654) (width 0.2) (layer "B.Cu") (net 6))
 (segment (start 149.51 43.1) (end 147.643654 43.1) (width 0.2) (layer "B.Cu") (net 6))
 (segment (start 143.64 58.93) (end 126.69 75.88) (width 0.2) (layer "B.Cu") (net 8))
 (segment (start 143.64 48.73) (end 143.64 58.93) (width 0.2) (layer "B.Cu") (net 8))
 (segment (start 148.12 44.25) (end 143.64 48.73) (width 0.2) (layer "B.Cu") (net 8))
 (segment (start 159.4 23) (end 159.4 56.5) (width 0.2) (layer "F.Cu") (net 9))
 (segment (start 158 56.5) (end 157.96 56.46) (width 0.2) (layer "F.Cu") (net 9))
 (segment (start 157.96 56.46) (end 146.11 56.46) (width 0.2) (layer "F.Cu") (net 9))
 (segment (start 159.4 56.5) (end 158 56.5) (width 0.2) (layer "F.Cu") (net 9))
 (segment (start 140.5 29) (end 140.5 23) (width 0.2) (layer "F.Cu") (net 9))
 (segment (start 140.5 23) (end 159.4 23) (width 0.2) (layer "F.Cu") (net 9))
 (segment (start 147.129899 55.5) (end 146.689899 55.06) (width 0.2) (layer "F.Cu") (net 5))
 (segment (start 143.04 29) (end 143.04 24.04) (width 0.2) (layer "F.Cu") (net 5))
 (segment (start 143.64 73.41) (end 146.11 75.88) (width 0.2) (layer "F.Cu") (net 5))
 (segment (start 159 55.5) (end 147.129899 55.5) (width 0.2) (layer "F.Cu") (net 5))
 (segment (start 146.689899 55.06) (end 145.44 55.06) (width 0.2) (layer "F.Cu") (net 5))
 (segment (start 159 24) (end 159 55.5) (width 0.2) (layer "F.Cu") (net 5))
 (segment (start 145.44 55.06) (end 143.64 56.86) (width 0.2) (layer "F.Cu") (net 5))
 (segment (start 143.04 24.04) (end 143 24) (width 0.2) (layer "F.Cu") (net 5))
 (segment (start 143 24) (end 159 24) (width 0.2) (layer "F.Cu") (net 5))
 (segment (start 143.64 56.86) (end 143.64 73.41) (width 0.2) (layer "F.Cu") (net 5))
 (segment (start 102 93.5) (end 124.85 93.5) (width 0.2) (layer "B.Cu") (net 11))
 (segment (start 124.85 93.5) (end 126.05 94.7) (width 0.2) (layer "B.Cu") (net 11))
 (segment (start 126.05 94.7) (end 126.05 99.7) (width 0.2) (layer "B.Cu") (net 11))
 (segment (start 102 31) (end 102 93.5) (width 0.2) (layer "B.Cu") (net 11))
 (segment (start 126.05 99.7) (end 124.75 101) (width 0.2) (layer "B.Cu") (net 11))
 (segment (start 148.12 29) (end 146.12 31) (width 0.2) (layer "B.Cu") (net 11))
 (segment (start 146.12 31) (end 102 31) (width 0.2) (layer "B.Cu") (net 11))
 (segment (start 145.58 29) (end 144.43 30.15) (width 0.2) (layer "B.Cu") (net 10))
 (segment (start 101.1 30.4) (end 101.1 94.6) (width 0.2) (layer "B.Cu") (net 10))
 (segment (start 105.5 96) (end 124.75 96) (width 0.2) (layer "B.Cu") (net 10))
 (segment (start 101.1 94.6) (end 101.5 95) (width 0.2) (layer "B.Cu") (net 10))
 (segment (start 104.5 95) (end 105.5 96) (width 0.2) (layer "B.Cu") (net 10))
 (segment (start 101.5 95) (end 104.5 95) (width 0.2) (layer "B.Cu") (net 10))
 (segment (start 101.35 30.15) (end 101.1 30.4) (width 0.2) (layer "B.Cu") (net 10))
 (segment (start 144.43 30.15) (end 101.35 30.15) (width 0.2) (layer "B.Cu") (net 10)))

